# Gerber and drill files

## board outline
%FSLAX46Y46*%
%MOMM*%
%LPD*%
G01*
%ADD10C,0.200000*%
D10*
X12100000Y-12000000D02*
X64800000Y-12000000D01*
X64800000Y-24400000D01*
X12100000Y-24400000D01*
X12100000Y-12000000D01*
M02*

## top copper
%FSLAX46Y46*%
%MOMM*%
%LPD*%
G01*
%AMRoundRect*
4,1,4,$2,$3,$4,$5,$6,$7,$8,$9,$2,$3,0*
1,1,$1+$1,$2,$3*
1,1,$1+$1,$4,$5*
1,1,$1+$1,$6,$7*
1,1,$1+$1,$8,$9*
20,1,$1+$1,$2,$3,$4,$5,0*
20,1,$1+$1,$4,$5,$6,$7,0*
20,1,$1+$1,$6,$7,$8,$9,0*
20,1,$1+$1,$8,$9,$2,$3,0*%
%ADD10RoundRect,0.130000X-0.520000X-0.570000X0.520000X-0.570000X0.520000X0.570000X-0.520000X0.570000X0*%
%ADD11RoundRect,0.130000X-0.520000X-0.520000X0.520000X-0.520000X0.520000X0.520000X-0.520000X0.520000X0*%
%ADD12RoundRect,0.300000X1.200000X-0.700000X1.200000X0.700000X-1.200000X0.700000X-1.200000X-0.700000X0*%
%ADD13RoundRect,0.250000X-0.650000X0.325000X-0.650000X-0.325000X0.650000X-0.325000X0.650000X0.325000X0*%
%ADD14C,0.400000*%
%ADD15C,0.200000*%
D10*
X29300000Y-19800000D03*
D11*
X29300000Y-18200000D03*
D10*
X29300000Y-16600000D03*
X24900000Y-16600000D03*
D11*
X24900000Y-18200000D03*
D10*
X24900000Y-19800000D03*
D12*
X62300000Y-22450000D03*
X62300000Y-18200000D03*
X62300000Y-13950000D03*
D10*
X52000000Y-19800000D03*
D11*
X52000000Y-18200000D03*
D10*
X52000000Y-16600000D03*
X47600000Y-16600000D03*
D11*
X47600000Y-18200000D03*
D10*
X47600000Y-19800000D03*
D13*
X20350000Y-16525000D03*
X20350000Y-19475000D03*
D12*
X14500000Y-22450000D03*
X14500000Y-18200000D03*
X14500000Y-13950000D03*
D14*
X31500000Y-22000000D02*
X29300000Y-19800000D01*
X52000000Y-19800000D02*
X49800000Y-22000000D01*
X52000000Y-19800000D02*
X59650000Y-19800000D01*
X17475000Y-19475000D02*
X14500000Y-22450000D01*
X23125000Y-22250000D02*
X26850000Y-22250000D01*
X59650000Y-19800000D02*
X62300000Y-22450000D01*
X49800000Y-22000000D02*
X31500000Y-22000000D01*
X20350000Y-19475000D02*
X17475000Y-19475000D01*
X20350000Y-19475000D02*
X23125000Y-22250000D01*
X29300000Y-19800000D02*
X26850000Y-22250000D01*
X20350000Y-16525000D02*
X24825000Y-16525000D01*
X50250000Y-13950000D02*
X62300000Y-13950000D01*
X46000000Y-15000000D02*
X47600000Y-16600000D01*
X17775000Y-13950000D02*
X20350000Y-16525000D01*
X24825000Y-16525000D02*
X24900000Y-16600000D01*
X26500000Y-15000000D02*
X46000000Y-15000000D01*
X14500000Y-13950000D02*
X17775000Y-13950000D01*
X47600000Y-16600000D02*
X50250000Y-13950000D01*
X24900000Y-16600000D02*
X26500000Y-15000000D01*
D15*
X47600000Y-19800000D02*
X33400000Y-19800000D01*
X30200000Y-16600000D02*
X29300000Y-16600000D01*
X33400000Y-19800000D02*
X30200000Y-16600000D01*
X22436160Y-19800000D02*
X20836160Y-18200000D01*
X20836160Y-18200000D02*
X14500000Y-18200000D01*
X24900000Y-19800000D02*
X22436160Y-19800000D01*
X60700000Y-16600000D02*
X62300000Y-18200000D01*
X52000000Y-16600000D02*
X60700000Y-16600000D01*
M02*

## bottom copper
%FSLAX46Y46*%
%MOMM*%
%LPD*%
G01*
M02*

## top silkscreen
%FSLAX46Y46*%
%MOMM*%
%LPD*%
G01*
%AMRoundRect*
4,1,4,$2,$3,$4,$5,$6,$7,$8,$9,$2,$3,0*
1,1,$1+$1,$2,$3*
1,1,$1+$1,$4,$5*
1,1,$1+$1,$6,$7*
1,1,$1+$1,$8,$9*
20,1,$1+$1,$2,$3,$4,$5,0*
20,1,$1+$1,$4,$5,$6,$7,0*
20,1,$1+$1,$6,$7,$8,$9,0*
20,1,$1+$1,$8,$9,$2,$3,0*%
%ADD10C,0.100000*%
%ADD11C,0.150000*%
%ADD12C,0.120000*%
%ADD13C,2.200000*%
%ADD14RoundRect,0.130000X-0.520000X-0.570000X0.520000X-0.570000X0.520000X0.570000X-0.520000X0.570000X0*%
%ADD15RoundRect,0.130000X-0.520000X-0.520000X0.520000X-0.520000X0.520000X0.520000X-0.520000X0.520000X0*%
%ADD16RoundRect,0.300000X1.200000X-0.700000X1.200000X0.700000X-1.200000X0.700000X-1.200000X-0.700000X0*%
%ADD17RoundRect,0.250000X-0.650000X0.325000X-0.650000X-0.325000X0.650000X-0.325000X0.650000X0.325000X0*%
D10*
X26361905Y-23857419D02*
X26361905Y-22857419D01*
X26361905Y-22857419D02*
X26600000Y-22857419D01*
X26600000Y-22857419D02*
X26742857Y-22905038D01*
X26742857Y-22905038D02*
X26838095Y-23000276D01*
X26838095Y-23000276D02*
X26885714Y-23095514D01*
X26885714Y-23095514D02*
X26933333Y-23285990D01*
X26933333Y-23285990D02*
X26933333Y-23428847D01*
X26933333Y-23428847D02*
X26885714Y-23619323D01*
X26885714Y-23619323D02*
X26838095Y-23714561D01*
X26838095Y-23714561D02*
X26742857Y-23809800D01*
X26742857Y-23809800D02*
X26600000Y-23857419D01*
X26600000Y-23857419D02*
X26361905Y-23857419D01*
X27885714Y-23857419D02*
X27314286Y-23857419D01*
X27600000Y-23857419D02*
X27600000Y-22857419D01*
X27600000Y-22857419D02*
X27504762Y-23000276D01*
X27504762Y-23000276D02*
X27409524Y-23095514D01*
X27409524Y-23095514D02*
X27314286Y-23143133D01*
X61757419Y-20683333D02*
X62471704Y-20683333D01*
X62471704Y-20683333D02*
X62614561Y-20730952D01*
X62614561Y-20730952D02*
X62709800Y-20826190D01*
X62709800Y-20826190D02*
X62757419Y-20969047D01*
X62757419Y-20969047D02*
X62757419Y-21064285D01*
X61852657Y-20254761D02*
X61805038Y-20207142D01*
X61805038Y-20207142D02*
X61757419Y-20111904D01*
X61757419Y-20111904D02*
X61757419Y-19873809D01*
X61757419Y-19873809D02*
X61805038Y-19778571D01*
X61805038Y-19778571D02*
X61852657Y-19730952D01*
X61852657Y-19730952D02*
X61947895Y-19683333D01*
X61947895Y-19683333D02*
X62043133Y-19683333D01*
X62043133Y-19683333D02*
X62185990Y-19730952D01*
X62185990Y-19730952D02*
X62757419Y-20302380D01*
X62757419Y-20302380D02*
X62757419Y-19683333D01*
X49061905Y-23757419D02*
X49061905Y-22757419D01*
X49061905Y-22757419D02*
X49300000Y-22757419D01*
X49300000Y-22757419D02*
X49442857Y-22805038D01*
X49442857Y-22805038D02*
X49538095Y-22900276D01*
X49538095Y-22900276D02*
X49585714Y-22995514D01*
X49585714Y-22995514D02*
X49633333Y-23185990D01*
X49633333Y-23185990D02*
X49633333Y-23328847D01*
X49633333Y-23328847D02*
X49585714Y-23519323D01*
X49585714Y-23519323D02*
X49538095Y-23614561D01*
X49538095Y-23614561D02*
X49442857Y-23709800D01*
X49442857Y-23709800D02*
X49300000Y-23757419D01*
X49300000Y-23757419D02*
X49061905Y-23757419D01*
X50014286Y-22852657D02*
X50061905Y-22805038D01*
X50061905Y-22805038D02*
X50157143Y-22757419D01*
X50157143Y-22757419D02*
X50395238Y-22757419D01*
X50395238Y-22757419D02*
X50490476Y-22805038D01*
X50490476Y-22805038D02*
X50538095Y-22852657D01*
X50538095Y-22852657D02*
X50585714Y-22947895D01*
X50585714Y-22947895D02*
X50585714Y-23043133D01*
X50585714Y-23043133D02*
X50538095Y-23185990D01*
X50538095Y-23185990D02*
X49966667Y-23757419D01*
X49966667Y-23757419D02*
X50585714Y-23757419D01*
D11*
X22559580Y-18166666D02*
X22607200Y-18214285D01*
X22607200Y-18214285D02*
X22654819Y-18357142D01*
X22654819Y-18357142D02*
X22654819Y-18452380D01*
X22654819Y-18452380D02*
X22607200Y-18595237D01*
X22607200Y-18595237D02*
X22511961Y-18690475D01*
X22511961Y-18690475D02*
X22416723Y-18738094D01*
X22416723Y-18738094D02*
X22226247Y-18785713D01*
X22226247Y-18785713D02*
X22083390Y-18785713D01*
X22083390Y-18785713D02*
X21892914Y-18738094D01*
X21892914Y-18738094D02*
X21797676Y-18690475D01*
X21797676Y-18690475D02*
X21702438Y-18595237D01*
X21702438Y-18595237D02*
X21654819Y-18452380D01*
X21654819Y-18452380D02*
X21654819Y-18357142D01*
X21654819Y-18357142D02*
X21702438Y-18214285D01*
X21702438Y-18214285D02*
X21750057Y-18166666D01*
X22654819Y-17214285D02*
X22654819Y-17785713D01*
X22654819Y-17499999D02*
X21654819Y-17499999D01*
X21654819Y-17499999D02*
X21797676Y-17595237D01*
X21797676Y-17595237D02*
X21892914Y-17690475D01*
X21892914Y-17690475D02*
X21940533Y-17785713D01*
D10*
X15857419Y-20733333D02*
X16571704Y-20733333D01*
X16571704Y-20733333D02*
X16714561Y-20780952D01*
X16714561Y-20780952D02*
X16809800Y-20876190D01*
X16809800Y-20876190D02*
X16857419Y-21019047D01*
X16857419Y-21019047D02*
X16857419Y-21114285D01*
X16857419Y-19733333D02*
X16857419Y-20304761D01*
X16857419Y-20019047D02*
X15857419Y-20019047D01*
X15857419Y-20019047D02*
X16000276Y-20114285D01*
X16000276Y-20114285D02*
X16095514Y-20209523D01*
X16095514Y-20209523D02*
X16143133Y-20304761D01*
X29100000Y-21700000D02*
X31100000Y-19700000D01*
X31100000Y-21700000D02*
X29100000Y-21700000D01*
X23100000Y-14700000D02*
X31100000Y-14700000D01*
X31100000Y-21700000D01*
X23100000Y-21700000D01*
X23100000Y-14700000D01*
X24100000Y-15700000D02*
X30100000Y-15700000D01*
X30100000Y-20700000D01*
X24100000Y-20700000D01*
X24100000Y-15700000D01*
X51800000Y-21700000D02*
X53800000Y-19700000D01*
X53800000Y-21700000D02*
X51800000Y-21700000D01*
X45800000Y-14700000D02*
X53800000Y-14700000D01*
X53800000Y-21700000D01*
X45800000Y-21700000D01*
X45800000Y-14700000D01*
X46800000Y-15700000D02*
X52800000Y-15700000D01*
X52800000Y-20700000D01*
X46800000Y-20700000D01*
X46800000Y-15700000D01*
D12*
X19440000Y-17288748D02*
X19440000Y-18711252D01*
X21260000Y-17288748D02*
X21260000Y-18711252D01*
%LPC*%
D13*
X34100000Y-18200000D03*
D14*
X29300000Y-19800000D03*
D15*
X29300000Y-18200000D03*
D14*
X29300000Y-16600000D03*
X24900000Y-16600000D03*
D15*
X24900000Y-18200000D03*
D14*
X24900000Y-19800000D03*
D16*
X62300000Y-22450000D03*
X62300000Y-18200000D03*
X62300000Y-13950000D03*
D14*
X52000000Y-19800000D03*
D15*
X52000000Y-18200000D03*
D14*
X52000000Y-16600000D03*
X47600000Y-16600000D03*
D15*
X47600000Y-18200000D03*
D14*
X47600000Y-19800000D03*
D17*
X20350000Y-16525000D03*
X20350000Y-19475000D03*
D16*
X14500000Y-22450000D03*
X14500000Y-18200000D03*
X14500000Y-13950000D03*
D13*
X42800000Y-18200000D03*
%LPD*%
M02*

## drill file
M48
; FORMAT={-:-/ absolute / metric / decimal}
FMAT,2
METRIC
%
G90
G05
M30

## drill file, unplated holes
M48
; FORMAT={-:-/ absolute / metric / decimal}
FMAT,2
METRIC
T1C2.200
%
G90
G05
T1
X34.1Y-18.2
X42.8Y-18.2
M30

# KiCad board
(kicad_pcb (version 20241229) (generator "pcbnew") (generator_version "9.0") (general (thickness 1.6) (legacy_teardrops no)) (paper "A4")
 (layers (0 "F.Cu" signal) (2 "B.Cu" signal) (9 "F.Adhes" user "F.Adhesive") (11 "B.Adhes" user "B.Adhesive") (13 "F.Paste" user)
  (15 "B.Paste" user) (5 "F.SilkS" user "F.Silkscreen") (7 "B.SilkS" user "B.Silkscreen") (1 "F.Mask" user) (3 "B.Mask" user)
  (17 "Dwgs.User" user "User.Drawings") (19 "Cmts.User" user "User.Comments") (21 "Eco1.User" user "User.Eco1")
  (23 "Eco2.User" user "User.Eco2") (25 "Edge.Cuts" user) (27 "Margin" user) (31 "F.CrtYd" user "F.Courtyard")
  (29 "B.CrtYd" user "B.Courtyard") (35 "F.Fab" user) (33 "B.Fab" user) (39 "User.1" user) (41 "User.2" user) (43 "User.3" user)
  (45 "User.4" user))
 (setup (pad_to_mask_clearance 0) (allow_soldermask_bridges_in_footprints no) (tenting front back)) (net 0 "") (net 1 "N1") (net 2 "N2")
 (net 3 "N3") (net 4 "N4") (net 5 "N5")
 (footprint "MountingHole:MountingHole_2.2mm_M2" (layer "F.Cu") (at 34.1 18.2)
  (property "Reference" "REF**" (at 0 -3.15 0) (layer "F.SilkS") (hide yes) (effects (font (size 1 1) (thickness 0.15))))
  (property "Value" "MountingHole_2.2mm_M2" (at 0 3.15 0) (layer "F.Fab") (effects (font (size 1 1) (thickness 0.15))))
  (pad "" np_thru_hole circle (at 0 0) (size 2.2 2.2) (drill 2.2) (layers "*.Cu" "*.Mask")))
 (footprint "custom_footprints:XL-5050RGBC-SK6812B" (layer "F.Cu") (at 27.1 18.2)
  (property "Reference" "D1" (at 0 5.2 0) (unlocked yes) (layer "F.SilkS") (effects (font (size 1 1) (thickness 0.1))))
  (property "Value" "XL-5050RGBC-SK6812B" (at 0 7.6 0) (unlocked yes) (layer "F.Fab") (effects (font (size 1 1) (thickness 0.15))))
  (fp_line (start 2 3.5) (end 4 1.5) (stroke (width 0.1) (type default)) (layer "F.SilkS"))
  (fp_line (start 4 3.5) (end 2 3.5) (stroke (width 0.1) (type default)) (layer "F.SilkS"))
  (fp_rect (start -4 -3.5) (end 4 3.5) (stroke (width 0.1) (type solid)) (fill no) (layer "F.SilkS"))
  (fp_rect (start -3 -2.5) (end 3 2.5) (stroke (width 0.1) (type solid)) (fill no) (layer "F.SilkS"))
  (pad "1" smd roundrect (at 2.2 1.6) (size 1.3 1.4) (layers "F.Cu" "F.Mask" "F.Paste") (roundrect_rratio 0.1) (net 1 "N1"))
  (pad "2" smd roundrect (at 2.2 0) (size 1.3 1.3) (layers "F.Cu" "F.Mask" "F.Paste") (roundrect_rratio 0.1))
  (pad "3" smd roundrect (at 2.2 -1.6) (size 1.3 1.4) (layers "F.Cu" "F.Mask" "F.Paste") (roundrect_rratio 0.1) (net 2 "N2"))
  (pad "4" smd roundrect (at -2.2 -1.6) (size 1.3 1.4) (layers "F.Cu" "F.Mask" "F.Paste") (roundrect_rratio 0.1) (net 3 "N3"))
  (pad "5" smd roundrect (at -2.2 0) (size 1.3 1.3) (layers "F.Cu" "F.Mask" "F.Paste") (roundrect_rratio 0.1))
  (pad "6" smd roundrect (at -2.2 1.6) (size 1.3 1.4) (layers "F.Cu" "F.Mask" "F.Paste") (roundrect_rratio 0.1) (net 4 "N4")))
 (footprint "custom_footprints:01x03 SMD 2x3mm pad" (layer "F.Cu") (at 62.3 18.2 90)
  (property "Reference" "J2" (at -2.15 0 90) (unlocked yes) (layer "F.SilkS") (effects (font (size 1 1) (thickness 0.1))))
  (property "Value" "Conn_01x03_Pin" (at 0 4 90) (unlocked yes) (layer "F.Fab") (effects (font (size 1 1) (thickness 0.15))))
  (pad "1" smd roundrect (at -4.25 0 90) (size 2 3) (layers "F.Cu" "F.Mask" "F.Paste") (roundrect_rratio 0.15) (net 1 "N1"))
  (pad "2" smd roundrect (at 0 0 90) (size 2 3) (layers "F.Cu" "F.Mask" "F.Paste") (roundrect_rratio 0.15) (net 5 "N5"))
  (pad "3" smd roundrect (at 4.25 0 90) (size 2 3) (layers "F.Cu" "F.Mask" "F.Paste") (roundrect_rratio 0.15) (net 3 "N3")))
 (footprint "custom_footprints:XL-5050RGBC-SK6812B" (layer "F.Cu") (at 49.8 18.2)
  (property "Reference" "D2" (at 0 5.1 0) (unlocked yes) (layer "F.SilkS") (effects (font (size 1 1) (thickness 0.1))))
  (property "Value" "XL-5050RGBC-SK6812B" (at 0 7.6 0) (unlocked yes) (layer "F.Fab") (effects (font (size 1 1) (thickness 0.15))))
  (fp_line (start 2 3.5) (end 4 1.5) (stroke (width 0.1) (type default)) (layer "F.SilkS"))
  (fp_line (start 4 3.5) (end 2 3.5) (stroke (width 0.1) (type default)) (layer "F.SilkS"))
  (fp_rect (start -4 -3.5) (end 4 3.5) (stroke (width 0.1) (type solid)) (fill no) (layer "F.SilkS"))
  (fp_rect (start -3 -2.5) (end 3 2.5) (stroke (width 0.1) (type solid)) (fill no) (layer "F.SilkS"))
  (pad "1" smd roundrect (at 2.2 1.6) (size 1.3 1.4) (layers "F.Cu" "F.Mask" "F.Paste") (roundrect_rratio 0.1) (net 1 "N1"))
  (pad "2" smd roundrect (at 2.2 0) (size 1.3 1.3) (layers "F.Cu" "F.Mask" "F.Paste") (roundrect_rratio 0.1))
  (pad "3" smd roundrect (at 2.2 -1.6) (size 1.3 1.4) (layers "F.Cu" "F.Mask" "F.Paste") (roundrect_rratio 0.1) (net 5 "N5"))
  (pad "4" smd roundrect (at -2.2 -1.6) (size 1.3 1.4) (layers "F.Cu" "F.Mask" "F.Paste") (roundrect_rratio 0.1) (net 3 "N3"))
  (pad "5" smd roundrect (at -2.2 0) (size 1.3 1.3) (layers "F.Cu" "F.Mask" "F.Paste") (roundrect_rratio 0.1))
  (pad "6" smd roundrect (at -2.2 1.6) (size 1.3 1.4) (layers "F.Cu" "F.Mask" "F.Paste") (roundrect_rratio 0.1) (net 2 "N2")))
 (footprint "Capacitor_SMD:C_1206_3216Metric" (layer "F.Cu") (at 20.35 18 -90)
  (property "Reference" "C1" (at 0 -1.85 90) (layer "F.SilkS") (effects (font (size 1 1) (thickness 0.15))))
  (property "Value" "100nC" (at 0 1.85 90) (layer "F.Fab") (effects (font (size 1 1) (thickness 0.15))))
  (fp_line (start -0.711252 0.91) (end 0.711252 0.91) (stroke (width 0.12) (type solid)) (layer "F.SilkS"))
  (fp_line (start -0.711252 -0.91) (end 0.711252 -0.91) (stroke (width 0.12) (type solid)) (layer "F.SilkS"))
  (pad "1" smd roundrect (at -1.475 0 270) (size 1.15 1.8) (layers "F.Cu" "F.Mask" "F.Paste") (roundrect_rratio 0.217391) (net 3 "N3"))
  (pad "2" smd roundrect (at 1.475 0 270) (size 1.15 1.8) (layers "F.Cu" "F.Mask" "F.Paste") (roundrect_rratio 0.217391) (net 1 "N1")))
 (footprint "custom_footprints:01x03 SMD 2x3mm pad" (layer "F.Cu") (at 14.5 18.2 90)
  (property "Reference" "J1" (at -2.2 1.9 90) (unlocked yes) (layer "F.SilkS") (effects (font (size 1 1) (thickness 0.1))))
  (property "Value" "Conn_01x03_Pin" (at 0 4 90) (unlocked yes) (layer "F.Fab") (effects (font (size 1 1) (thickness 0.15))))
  (pad "1" smd roundrect (at -4.25 0 90) (size 2 3) (layers "F.Cu" "F.Mask" "F.Paste") (roundrect_rratio 0.15) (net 1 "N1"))
  (pad "2" smd roundrect (at 0 0 90) (size 2 3) (layers "F.Cu" "F.Mask" "F.Paste") (roundrect_rratio 0.15) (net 4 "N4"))
  (pad "3" smd roundrect (at 4.25 0 90) (size 2 3) (layers "F.Cu" "F.Mask" "F.Paste") (roundrect_rratio 0.15) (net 3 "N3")))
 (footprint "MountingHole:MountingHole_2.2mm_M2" (layer "F.Cu") (at 42.8 18.2)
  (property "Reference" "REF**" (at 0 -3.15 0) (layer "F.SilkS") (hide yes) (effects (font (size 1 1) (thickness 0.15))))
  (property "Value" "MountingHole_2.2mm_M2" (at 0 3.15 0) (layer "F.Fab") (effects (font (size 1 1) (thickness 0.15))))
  (pad "" np_thru_hole circle (at 0 0) (size 2.2 2.2) (drill 2.2) (layers "*.Cu" "*.Mask")))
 (gr_rect (start 12.1 12) (end 64.8 24.4) (stroke (width 0.2) (type default)) (fill no) (layer "Edge.Cuts"))
 (segment (start 31.5 22) (end 29.3 19.8) (width 0.4) (layer "F.Cu") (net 1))
 (segment (start 52 19.8) (end 49.8 22) (width 0.4) (layer "F.Cu") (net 1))
 (segment (start 52 19.8) (end 59.65 19.8) (width 0.4) (layer "F.Cu") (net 1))
 (segment (start 17.475 19.475) (end 14.5 22.45) (width 0.4) (layer "F.Cu") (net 1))
 (segment (start 23.125 22.25) (end 26.85 22.25) (width 0.4) (layer "F.Cu") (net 1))
 (segment (start 59.65 19.8) (end 62.3 22.45) (width 0.4) (layer "F.Cu") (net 1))
 (segment (start 49.8 22) (end 31.5 22) (width 0.4) (layer "F.Cu") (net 1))
 (segment (start 20.35 19.475) (end 17.475 19.475) (width 0.4) (layer "F.Cu") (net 1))
 (segment (start 20.35 19.475) (end 23.125 22.25) (width 0.4) (layer "F.Cu") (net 1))
 (segment (start 29.3 19.8) (end 26.85 22.25) (width 0.4) (layer "F.Cu") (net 1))
 (segment (start 20.35 16.525) (end 24.825 16.525) (width 0.4) (layer "F.Cu") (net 3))
 (segment (start 50.25 13.95) (end 62.3 13.95) (width 0.4) (layer "F.Cu") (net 3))
 (segment (start 46 15) (end 47.6 16.6) (width 0.4) (layer "F.Cu") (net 3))
 (segment (start 17.775 13.95) (end 20.35 16.525) (width 0.4) (layer "F.Cu") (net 3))
 (segment (start 24.825 16.525) (end 24.9 16.6) (width 0.4) (layer "F.Cu") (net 3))
 (segment (start 26.5 15) (end 46 15) (width 0.4) (layer "F.Cu") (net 3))
 (segment (start 14.5 13.95) (end 17.775 13.95) (width 0.4) (layer "F.Cu") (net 3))
 (segment (start 47.6 16.6) (end 50.25 13.95) (width 0.4) (layer "F.Cu") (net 3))
 (segment (start 24.9 16.6) (end 26.5 15) (width 0.4) (layer "F.Cu") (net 3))
 (segment (start 47.6 19.8) (end 33.4 19.8) (width 0.2) (layer "F.Cu") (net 2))
 (segment (start 30.2 16.6) (end 29.3 16.6) (width 0.2) (layer "F.Cu") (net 2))
 (segment (start 33.4 19.8) (end 30.2 16.6) (width 0.2) (layer "F.Cu") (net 2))
 (segment (start 22.43616 19.8) (end 20.83616 18.2) (width 0.2) (layer "F.Cu") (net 4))
 (segment (start 20.83616 18.2) (end 14.5 18.2) (width 0.2) (layer "F.Cu") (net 4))
 (segment (start 24.9 19.8) (end 22.43616 19.8) (width 0.2) (layer "F.Cu") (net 4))
 (segment (start 60.7 16.6) (end 62.3 18.2) (width 0.2) (layer "F.Cu") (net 5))
 (segment (start 52 16.6) (end 60.7 16.6) (width 0.2) (layer "F.Cu") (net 5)))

